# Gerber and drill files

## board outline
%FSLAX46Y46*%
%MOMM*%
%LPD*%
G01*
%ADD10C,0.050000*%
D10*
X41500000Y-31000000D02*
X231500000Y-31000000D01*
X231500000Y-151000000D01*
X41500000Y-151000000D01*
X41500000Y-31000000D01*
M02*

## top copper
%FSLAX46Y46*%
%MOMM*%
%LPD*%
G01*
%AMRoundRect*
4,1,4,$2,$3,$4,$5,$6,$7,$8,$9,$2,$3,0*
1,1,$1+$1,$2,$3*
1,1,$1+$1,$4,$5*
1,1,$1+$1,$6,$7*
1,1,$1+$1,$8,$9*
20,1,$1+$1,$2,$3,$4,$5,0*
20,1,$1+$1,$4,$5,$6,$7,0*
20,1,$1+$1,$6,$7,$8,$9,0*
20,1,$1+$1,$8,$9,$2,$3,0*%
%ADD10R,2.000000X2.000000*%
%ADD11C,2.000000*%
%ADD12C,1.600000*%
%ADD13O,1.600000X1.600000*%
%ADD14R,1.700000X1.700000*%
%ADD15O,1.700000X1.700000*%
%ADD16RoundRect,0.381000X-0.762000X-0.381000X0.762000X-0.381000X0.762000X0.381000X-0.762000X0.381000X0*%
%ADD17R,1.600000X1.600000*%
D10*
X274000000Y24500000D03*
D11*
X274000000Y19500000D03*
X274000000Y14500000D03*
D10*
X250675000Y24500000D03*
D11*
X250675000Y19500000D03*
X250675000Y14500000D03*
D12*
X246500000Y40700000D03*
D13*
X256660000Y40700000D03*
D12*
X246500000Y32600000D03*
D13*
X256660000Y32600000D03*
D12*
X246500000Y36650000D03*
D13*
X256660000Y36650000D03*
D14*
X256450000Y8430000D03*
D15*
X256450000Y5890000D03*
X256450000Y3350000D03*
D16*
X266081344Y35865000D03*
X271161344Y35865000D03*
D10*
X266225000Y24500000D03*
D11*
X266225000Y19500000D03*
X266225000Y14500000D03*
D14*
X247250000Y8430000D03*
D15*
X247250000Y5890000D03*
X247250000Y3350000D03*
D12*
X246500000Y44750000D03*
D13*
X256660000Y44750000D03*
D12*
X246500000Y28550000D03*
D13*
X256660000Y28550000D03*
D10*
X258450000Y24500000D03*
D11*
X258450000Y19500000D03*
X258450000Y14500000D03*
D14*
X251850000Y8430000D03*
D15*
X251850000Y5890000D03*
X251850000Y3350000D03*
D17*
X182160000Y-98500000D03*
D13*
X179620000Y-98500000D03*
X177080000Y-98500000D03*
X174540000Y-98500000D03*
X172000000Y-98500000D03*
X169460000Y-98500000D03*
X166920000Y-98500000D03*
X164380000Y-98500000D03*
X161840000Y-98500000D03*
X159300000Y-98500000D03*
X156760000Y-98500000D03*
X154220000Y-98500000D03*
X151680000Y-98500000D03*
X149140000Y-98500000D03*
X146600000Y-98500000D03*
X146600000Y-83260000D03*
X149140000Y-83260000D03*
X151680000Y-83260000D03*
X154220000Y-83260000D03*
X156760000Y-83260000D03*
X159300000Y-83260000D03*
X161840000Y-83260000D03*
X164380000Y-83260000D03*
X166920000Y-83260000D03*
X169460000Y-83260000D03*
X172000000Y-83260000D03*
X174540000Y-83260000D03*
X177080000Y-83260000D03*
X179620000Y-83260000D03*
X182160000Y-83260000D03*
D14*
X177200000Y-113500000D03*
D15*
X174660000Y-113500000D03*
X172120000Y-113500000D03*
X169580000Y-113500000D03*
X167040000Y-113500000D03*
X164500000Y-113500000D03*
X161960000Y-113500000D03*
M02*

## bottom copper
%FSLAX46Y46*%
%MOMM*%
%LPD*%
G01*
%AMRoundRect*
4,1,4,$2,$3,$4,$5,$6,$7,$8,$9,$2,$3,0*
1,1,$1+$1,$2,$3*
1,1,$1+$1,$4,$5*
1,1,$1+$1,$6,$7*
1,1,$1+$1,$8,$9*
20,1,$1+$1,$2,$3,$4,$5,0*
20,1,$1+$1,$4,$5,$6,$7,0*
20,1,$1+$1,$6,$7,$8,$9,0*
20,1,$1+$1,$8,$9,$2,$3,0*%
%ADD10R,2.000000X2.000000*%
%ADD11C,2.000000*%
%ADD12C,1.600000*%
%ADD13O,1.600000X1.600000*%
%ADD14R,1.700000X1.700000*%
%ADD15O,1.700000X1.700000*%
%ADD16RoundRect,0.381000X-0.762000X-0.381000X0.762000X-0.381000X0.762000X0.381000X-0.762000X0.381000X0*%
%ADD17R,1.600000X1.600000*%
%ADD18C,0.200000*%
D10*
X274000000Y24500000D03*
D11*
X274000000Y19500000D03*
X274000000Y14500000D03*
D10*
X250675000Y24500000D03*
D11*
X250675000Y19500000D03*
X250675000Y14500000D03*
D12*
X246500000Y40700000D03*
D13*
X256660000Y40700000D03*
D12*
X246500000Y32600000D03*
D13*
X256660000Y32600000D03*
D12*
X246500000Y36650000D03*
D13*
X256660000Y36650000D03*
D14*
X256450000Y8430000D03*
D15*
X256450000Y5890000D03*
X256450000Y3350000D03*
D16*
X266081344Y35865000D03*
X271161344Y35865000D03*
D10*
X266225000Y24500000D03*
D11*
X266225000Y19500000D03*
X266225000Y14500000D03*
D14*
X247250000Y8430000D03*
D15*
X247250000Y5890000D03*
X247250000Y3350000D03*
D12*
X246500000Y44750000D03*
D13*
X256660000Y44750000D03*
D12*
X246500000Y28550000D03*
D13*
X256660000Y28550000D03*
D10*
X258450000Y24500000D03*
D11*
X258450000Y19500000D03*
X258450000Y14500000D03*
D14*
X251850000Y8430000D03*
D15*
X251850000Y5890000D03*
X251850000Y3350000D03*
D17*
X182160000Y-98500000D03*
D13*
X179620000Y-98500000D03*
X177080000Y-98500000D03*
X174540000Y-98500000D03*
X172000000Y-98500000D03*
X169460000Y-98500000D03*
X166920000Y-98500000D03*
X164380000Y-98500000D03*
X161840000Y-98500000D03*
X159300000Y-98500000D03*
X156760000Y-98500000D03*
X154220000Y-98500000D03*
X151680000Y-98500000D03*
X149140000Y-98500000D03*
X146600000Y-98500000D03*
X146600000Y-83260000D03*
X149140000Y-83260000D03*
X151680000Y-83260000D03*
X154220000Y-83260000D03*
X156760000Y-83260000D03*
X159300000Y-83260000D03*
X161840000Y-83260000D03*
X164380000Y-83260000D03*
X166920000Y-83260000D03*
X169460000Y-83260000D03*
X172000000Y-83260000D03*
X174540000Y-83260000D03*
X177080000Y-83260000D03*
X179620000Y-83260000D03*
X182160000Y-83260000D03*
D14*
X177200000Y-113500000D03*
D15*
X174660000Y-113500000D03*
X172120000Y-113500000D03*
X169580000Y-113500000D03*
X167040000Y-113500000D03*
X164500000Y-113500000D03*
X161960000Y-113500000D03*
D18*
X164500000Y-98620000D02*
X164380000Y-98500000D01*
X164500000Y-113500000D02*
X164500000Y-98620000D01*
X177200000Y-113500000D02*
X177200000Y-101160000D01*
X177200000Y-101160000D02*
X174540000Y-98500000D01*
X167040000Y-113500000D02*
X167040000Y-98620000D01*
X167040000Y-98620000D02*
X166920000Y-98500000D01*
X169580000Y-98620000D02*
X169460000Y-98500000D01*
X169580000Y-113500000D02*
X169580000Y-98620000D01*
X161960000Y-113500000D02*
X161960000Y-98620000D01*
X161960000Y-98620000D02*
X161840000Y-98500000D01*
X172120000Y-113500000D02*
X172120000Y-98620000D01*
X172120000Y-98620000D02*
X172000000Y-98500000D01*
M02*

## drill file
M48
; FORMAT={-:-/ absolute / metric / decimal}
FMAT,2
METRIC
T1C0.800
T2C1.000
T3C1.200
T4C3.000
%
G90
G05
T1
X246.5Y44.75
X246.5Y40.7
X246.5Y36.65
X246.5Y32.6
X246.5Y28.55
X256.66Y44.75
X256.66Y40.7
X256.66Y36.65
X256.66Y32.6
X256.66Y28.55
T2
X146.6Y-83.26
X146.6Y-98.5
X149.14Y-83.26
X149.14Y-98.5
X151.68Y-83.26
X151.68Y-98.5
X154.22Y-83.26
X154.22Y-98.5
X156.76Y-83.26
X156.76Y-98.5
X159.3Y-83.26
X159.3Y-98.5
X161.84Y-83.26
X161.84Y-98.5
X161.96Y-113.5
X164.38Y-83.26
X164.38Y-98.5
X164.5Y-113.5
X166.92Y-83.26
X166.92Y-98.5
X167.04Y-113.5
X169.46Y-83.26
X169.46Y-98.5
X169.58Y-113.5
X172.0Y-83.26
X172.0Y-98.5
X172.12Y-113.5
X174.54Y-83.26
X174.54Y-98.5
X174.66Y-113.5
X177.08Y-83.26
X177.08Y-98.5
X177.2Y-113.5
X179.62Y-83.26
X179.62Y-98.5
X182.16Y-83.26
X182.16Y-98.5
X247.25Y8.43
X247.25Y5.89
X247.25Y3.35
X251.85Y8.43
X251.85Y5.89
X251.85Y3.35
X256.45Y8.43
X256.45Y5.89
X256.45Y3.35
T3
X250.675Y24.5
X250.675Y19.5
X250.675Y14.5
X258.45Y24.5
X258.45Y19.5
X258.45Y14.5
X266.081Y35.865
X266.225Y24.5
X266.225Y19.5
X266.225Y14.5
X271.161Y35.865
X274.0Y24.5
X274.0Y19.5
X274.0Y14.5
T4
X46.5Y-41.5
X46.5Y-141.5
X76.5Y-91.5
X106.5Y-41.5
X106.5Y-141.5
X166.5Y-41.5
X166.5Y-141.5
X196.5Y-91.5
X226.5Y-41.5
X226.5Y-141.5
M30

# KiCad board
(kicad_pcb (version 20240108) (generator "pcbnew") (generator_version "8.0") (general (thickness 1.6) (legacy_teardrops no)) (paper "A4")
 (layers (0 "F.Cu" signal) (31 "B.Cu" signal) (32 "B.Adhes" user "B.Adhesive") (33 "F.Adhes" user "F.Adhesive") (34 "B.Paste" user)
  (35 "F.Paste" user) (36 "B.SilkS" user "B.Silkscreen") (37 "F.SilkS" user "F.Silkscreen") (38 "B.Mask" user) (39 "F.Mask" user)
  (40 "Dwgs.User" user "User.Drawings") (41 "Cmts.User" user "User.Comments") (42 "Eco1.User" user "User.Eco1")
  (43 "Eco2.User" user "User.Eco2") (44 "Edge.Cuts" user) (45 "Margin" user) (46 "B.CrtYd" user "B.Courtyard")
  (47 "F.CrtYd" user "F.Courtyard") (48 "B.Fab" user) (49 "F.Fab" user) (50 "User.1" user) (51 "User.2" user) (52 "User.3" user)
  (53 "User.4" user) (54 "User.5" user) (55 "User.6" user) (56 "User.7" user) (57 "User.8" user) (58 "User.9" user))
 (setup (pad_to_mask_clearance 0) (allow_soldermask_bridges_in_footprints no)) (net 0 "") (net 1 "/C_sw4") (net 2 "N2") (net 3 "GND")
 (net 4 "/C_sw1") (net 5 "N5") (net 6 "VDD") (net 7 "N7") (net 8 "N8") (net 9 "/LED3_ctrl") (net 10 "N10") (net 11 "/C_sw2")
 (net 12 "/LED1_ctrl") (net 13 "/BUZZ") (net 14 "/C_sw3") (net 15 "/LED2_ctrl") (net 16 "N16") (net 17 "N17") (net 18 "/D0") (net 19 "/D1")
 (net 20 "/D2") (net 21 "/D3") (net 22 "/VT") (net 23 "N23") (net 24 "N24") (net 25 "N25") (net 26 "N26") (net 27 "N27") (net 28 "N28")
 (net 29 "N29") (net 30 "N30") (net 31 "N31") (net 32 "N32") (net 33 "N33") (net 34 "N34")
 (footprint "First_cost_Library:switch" (layer "F.Cu") (at 269 -11.5)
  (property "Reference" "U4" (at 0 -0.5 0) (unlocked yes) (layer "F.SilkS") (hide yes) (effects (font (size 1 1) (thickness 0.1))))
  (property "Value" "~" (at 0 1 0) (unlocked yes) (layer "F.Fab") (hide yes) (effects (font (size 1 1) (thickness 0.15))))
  (pad "1" thru_hole rect (at 5 -13) (size 2 2) (drill 1.2) (layers "*.Cu" "*.Mask") (remove_unused_layers no) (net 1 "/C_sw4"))
  (pad "2" thru_hole circle (at 5 -8) (size 2 2) (drill 1.2) (layers "*.Cu" "*.Mask") (remove_unused_layers no) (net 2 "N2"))
  (pad "3" thru_hole circle (at 5 -3) (size 2 2) (drill 1.2) (layers "*.Cu" "*.Mask") (remove_unused_layers no) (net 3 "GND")))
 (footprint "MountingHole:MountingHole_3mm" (layer "F.Cu") (at 196.5 91.5)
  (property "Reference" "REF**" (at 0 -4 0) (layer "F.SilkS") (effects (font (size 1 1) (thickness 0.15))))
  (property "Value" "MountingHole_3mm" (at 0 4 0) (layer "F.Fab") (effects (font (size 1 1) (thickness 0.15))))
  (pad "" np_thru_hole circle (at 0 0) (size 3 3) (drill 3) (layers "*.Cu" "*.Mask")))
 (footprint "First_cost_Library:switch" (layer "F.Cu") (at 245.675 -11.5)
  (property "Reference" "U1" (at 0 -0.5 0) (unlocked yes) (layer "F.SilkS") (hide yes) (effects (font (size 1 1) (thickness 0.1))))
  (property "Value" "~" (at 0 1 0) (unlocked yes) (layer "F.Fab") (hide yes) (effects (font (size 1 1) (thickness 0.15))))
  (pad "1" thru_hole rect (at 5 -13) (size 2 2) (drill 1.2) (layers "*.Cu" "*.Mask") (remove_unused_layers no) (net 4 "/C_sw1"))
  (pad "2" thru_hole circle (at 5 -8) (size 2 2) (drill 1.2) (layers "*.Cu" "*.Mask") (remove_unused_layers no) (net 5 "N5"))
  (pad "3" thru_hole circle (at 5 -3) (size 2 2) (drill 1.2) (layers "*.Cu" "*.Mask") (remove_unused_layers no) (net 3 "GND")))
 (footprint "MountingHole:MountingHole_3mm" (layer "F.Cu") (at 76.5 91.5)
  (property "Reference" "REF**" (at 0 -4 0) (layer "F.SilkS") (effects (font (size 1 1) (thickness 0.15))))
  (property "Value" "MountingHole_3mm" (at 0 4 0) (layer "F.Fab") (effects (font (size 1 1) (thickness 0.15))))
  (pad "" np_thru_hole circle (at 0 0) (size 3 3) (drill 3) (layers "*.Cu" "*.Mask")))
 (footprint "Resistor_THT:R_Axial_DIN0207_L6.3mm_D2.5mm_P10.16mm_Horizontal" (layer "F.Cu") (at 246.5 -40.7)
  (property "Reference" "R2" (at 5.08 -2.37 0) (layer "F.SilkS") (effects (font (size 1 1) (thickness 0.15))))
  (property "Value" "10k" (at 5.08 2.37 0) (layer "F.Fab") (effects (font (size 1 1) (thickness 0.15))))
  (pad "1" thru_hole circle (at 0 0) (size 1.6 1.6) (drill 0.8) (layers "*.Cu" "*.Mask") (remove_unused_layers no) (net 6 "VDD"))
  (pad "2" thru_hole oval (at 10.16 0) (size 1.6 1.6) (drill 0.8) (layers "*.Cu" "*.Mask") (remove_unused_layers no) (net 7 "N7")))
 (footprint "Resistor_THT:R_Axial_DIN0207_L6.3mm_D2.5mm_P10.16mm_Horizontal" (layer "F.Cu") (at 246.5 -32.6)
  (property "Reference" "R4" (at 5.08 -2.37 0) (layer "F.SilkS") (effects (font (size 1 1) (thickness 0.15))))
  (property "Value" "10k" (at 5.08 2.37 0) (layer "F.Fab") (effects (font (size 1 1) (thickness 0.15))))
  (pad "1" thru_hole circle (at 0 0) (size 1.6 1.6) (drill 0.8) (layers "*.Cu" "*.Mask") (remove_unused_layers no) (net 6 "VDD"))
  (pad "2" thru_hole oval (at 10.16 0) (size 1.6 1.6) (drill 0.8) (layers "*.Cu" "*.Mask") (remove_unused_layers no) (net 2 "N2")))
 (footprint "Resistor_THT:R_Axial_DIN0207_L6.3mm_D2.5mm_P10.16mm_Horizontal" (layer "F.Cu") (at 246.5 -36.65)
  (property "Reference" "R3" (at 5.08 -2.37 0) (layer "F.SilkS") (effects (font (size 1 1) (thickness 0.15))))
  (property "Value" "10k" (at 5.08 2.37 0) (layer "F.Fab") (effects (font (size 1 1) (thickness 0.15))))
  (pad "1" thru_hole circle (at 0 0) (size 1.6 1.6) (drill 0.8) (layers "*.Cu" "*.Mask") (remove_unused_layers no) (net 6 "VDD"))
  (pad "2" thru_hole oval (at 10.16 0) (size 1.6 1.6) (drill 0.8) (layers "*.Cu" "*.Mask") (remove_unused_layers no) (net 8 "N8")))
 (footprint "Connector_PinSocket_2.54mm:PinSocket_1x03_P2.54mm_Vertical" (layer "F.Cu") (at 256.45 -8.43)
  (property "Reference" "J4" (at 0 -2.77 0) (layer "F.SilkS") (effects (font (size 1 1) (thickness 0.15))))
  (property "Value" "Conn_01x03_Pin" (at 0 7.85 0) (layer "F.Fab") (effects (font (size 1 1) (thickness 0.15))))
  (pad "1" thru_hole rect (at 0 0) (size 1.7 1.7) (drill 1) (layers "*.Cu" "*.Mask") (remove_unused_layers no) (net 6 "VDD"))
  (pad "2" thru_hole oval (at 0 2.54) (size 1.7 1.7) (drill 1) (layers "*.Cu" "*.Mask") (remove_unused_layers no) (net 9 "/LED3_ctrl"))
  (pad "3" thru_hole oval (at 0 5.08) (size 1.7 1.7) (drill 1) (layers "*.Cu" "*.Mask") (remove_unused_layers no) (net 3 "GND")))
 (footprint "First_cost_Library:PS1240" (layer "F.Cu") (at 268.621344 -46.025)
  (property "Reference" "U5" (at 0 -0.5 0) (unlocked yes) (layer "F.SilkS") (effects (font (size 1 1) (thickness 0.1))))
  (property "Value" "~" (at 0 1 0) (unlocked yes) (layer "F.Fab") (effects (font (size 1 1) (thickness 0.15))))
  (pad "1" thru_hole roundrect (at -2.54 10.16) (size 2.286 1.524) (drill 1.2) (layers "*.Cu" "*.Mask") (remove_unused_layers no)
   (roundrect_rratio 0.25) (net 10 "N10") (thermal_bridge_angle 45))
  (pad "2" thru_hole roundrect (at 2.54 10.16) (size 2.286 1.524) (drill 1.2) (layers "*.Cu" "*.Mask") (remove_unused_layers no)
   (roundrect_rratio 0.25) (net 3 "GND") (thermal_bridge_angle 45)))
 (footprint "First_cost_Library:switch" (layer "F.Cu") (at 261.225 -11.5)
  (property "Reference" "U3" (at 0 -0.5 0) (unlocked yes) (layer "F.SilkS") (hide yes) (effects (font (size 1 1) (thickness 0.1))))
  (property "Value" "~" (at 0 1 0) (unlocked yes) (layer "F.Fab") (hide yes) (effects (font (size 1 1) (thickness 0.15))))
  (pad "1" thru_hole rect (at 5 -13) (size 2 2) (drill 1.2) (layers "*.Cu" "*.Mask") (remove_unused_layers no) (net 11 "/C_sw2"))
  (pad "2" thru_hole circle (at 5 -8) (size 2 2) (drill 1.2) (layers "*.Cu" "*.Mask") (remove_unused_layers no) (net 8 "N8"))
  (pad "3" thru_hole circle (at 5 -3) (size 2 2) (drill 1.2) (layers "*.Cu" "*.Mask") (remove_unused_layers no) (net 3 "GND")))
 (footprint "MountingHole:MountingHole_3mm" (layer "F.Cu") (at 166.5 141.5)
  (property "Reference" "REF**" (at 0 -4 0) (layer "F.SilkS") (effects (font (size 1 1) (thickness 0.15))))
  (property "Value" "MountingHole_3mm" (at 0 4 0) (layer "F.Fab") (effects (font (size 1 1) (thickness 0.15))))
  (pad "" np_thru_hole circle (at 0 0) (size 3 3) (drill 3) (layers "*.Cu" "*.Mask")))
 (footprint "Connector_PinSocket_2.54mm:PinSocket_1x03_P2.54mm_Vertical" (layer "F.Cu") (at 247.25 -8.43)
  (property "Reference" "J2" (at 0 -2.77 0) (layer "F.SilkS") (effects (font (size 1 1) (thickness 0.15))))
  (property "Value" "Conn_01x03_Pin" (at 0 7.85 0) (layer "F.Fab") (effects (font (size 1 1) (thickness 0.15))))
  (pad "1" thru_hole rect (at 0 0) (size 1.7 1.7) (drill 1) (layers "*.Cu" "*.Mask") (remove_unused_layers no) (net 6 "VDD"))
  (pad "2" thru_hole oval (at 0 2.54) (size 1.7 1.7) (drill 1) (layers "*.Cu" "*.Mask") (remove_unused_layers no) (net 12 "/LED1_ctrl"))
  (pad "3" thru_hole oval (at 0 5.08) (size 1.7 1.7) (drill 1) (layers "*.Cu" "*.Mask") (remove_unused_layers no) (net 3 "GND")))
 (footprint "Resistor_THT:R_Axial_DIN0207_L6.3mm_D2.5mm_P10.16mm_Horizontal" (layer "F.Cu") (at 246.5 -44.75)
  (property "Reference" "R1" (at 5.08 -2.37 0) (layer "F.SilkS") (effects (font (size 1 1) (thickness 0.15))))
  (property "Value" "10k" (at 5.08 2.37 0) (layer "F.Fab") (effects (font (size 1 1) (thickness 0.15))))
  (pad "1" thru_hole circle (at 0 0) (size 1.6 1.6) (drill 0.8) (layers "*.Cu" "*.Mask") (remove_unused_layers no) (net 6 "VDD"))
  (pad "2" thru_hole oval (at 10.16 0) (size 1.6 1.6) (drill 0.8) (layers "*.Cu" "*.Mask") (remove_unused_layers no) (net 5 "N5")))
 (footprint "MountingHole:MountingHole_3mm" (layer "F.Cu") (at 106.5 141.5)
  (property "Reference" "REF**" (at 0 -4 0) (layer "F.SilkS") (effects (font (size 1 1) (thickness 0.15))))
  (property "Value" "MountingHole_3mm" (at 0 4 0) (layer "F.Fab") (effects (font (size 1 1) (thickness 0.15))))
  (pad "" np_thru_hole circle (at 0 0) (size 3 3) (drill 3) (layers "*.Cu" "*.Mask")))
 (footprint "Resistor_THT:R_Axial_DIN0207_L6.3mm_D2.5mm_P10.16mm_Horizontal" (layer "F.Cu") (at 246.5 -28.55)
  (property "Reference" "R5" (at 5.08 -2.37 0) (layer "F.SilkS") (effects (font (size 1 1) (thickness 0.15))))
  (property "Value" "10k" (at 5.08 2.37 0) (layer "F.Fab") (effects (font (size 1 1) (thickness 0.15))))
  (pad "1" thru_hole circle (at 0 0) (size 1.6 1.6) (drill 0.8) (layers "*.Cu" "*.Mask") (remove_unused_layers no) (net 10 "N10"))
  (pad "2" thru_hole oval (at 10.16 0) (size 1.6 1.6) (drill 0.8) (layers "*.Cu" "*.Mask") (remove_unused_layers no) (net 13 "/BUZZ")))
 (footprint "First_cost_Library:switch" (layer "F.Cu") (at 253.45 -11.5)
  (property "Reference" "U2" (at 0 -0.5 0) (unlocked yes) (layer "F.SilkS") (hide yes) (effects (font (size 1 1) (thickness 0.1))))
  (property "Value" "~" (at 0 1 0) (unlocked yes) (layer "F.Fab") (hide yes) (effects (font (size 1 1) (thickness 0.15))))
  (pad "1" thru_hole rect (at 5 -13) (size 2 2) (drill 1.2) (layers "*.Cu" "*.Mask") (remove_unused_layers no) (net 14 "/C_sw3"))
  (pad "2" thru_hole circle (at 5 -8) (size 2 2) (drill 1.2) (layers "*.Cu" "*.Mask") (remove_unused_layers no) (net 7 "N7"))
  (pad "3" thru_hole circle (at 5 -3) (size 2 2) (drill 1.2) (layers "*.Cu" "*.Mask") (remove_unused_layers no) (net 3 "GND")))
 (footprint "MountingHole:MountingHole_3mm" (layer "F.Cu") (at 226.5 41.5)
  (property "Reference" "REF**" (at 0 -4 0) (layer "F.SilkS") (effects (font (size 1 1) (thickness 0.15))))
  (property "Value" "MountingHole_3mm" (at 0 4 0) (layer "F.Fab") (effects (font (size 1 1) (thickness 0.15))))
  (pad "" np_thru_hole circle (at 0 0) (size 3 3) (drill 3) (layers "*.Cu" "*.Mask")))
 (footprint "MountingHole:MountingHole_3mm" (layer "F.Cu") (at 166.5 41.5)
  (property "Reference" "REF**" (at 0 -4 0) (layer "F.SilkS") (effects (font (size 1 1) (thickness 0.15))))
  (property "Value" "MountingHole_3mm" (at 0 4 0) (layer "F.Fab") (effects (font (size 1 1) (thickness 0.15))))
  (pad "" np_thru_hole circle (at 0 0) (size 3 3) (drill 3) (layers "*.Cu" "*.Mask")))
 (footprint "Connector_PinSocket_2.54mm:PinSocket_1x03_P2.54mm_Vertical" (layer "F.Cu") (at 251.85 -8.43)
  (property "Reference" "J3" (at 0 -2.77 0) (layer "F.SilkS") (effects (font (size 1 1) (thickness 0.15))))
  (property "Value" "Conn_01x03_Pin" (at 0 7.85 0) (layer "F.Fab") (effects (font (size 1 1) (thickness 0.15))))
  (pad "1" thru_hole rect (at 0 0) (size 1.7 1.7) (drill 1) (layers "*.Cu" "*.Mask") (remove_unused_layers no) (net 6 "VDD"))
  (pad "2" thru_hole oval (at 0 2.54) (size 1.7 1.7) (drill 1) (layers "*.Cu" "*.Mask") (remove_unused_layers no) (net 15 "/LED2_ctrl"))
  (pad "3" thru_hole oval (at 0 5.08) (size 1.7 1.7) (drill 1) (layers "*.Cu" "*.Mask") (remove_unused_layers no) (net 3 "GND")))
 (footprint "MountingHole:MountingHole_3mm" (layer "F.Cu") (at 46.5 141.5)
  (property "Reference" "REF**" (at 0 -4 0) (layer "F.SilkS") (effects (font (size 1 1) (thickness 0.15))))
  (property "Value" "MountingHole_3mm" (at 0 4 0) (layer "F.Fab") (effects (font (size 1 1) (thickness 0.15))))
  (pad "" np_thru_hole circle (at 0 0) (size 3 3) (drill 3) (layers "*.Cu" "*.Mask")))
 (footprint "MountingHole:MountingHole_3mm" (layer "F.Cu") (at 46.5 41.5)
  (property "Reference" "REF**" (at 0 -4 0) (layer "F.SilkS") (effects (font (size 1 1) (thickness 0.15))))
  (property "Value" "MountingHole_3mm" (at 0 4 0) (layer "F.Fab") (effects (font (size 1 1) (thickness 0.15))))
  (pad "" np_thru_hole circle (at 0 0) (size 3 3) (drill 3) (layers "*.Cu" "*.Mask")))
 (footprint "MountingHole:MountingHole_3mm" (layer "F.Cu") (at 226.5 141.5)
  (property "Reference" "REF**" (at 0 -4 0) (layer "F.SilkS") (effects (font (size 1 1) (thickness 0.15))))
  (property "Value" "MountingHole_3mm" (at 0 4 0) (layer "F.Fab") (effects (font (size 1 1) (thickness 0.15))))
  (pad "" np_thru_hole circle (at 0 0) (size 3 3) (drill 3) (layers "*.Cu" "*.Mask")))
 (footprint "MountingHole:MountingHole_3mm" (layer "F.Cu") (at 106.5 41.5)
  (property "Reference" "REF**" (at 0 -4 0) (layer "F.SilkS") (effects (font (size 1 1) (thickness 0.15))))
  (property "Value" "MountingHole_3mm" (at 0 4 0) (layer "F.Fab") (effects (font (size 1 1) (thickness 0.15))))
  (pad "" np_thru_hole circle (at 0 0) (size 3 3) (drill 3) (layers "*.Cu" "*.Mask")))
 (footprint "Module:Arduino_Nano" (layer "B.Cu") (at 182.16 98.5 90)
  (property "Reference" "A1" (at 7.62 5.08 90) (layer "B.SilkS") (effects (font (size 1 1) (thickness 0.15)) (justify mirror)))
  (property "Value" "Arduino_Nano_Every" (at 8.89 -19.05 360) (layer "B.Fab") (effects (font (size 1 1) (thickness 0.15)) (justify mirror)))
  (pad "1" thru_hole rect (at 0 0 90) (size 1.6 1.6) (drill 1) (layers "*.Cu" "*.Mask") (remove_unused_layers no) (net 13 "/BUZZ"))
  (pad "2" thru_hole oval (at 0 -2.54 90) (size 1.6 1.6) (drill 1) (layers "*.Cu" "*.Mask") (remove_unused_layers no) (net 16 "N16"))
  (pad "3" thru_hole oval (at 0 -5.08 90) (size 1.6 1.6) (drill 1) (layers "*.Cu" "*.Mask") (remove_unused_layers no) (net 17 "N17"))
  (pad "4" thru_hole oval (at 0 -7.62 90) (size 1.6 1.6) (drill 1) (layers "*.Cu" "*.Mask") (remove_unused_layers no) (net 3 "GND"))
  (pad "5" thru_hole oval (at 0 -10.16 90) (size 1.6 1.6) (drill 1) (layers "*.Cu" "*.Mask") (remove_unused_layers no) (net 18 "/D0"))
  (pad "6" thru_hole oval (at 0 -12.7 90) (size 1.6 1.6) (drill 1) (layers "*.Cu" "*.Mask") (remove_unused_layers no) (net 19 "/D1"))
  (pad "7" thru_hole oval (at 0 -15.24 90) (size 1.6 1.6) (drill 1) (layers "*.Cu" "*.Mask") (remove_unused_layers no) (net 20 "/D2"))
  (pad "8" thru_hole oval (at 0 -17.78 90) (size 1.6 1.6) (drill 1) (layers "*.Cu" "*.Mask") (remove_unused_layers no) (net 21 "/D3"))
  (pad "9" thru_hole oval (at 0 -20.32 90) (size 1.6 1.6) (drill 1) (layers "*.Cu" "*.Mask") (remove_unused_layers no) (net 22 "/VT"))
  (pad "10" thru_hole oval (at 0 -22.86 90) (size 1.6 1.6) (drill 1) (layers "*.Cu" "*.Mask") (remove_unused_layers no) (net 4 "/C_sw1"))
  (pad "11" thru_hole oval (at 0 -25.4 90) (size 1.6 1.6) (drill 1) (layers "*.Cu" "*.Mask") (remove_unused_layers no) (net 11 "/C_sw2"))
  (pad "12" thru_hole oval (at 0 -27.94 90) (size 1.6 1.6) (drill 1) (layers "*.Cu" "*.Mask") (remove_unused_layers no) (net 14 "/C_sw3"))
  (pad "13" thru_hole oval (at 0 -30.48 90) (size 1.6 1.6) (drill 1) (layers "*.Cu" "*.Mask") (remove_unused_layers no) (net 1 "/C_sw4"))
  (pad "14" thru_hole oval (at 0 -33.02 90) (size 1.6 1.6) (drill 1) (layers "*.Cu" "*.Mask") (remove_unused_layers no)
   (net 12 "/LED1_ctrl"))
  (pad "15" thru_hole oval (at 0 -35.56 90) (size 1.6 1.6) (drill 1) (layers "*.Cu" "*.Mask") (remove_unused_layers no)
   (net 15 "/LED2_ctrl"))
  (pad "16" thru_hole oval (at 15.24 -35.56 90) (size 1.6 1.6) (drill 1) (layers "*.Cu" "*.Mask") (remove_unused_layers no)
   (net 9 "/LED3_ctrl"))
  (pad "17" thru_hole oval (at 15.24 -33.02 90) (size 1.6 1.6) (drill 1) (layers "*.Cu" "*.Mask") (remove_unused_layers no) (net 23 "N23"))
  (pad "18" thru_hole oval (at 15.24 -30.48 90) (size 1.6 1.6) (drill 1) (layers "*.Cu" "*.Mask") (remove_unused_layers no) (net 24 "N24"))
  (pad "19" thru_hole oval (at 15.24 -27.94 90) (size 1.6 1.6) (drill 1) (layers "*.Cu" "*.Mask") (remove_unused_layers no) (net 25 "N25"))
  (pad "20" thru_hole oval (at 15.24 -25.4 90) (size 1.6 1.6) (drill 1) (layers "*.Cu" "*.Mask") (remove_unused_layers no) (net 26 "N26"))
  (pad "21" thru_hole oval (at 15.24 -22.86 90) (size 1.6 1.6) (drill 1) (layers "*.Cu" "*.Mask") (remove_unused_layers no) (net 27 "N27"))
  (pad "22" thru_hole oval (at 15.24 -20.32 90) (size 1.6 1.6) (drill 1) (layers "*.Cu" "*.Mask") (remove_unused_layers no) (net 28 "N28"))
  (pad "23" thru_hole oval (at 15.24 -17.78 90) (size 1.6 1.6) (drill 1) (layers "*.Cu" "*.Mask") (remove_unused_layers no) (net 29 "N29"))
  (pad "24" thru_hole oval (at 15.24 -15.24 90) (size 1.6 1.6) (drill 1) (layers "*.Cu" "*.Mask") (remove_unused_layers no) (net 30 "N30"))
  (pad "25" thru_hole oval (at 15.24 -12.7 90) (size 1.6 1.6) (drill 1) (layers "*.Cu" "*.Mask") (remove_unused_layers no) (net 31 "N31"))
  (pad "26" thru_hole oval (at 15.24 -10.16 90) (size 1.6 1.6) (drill 1) (layers "*.Cu" "*.Mask") (remove_unused_layers no) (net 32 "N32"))
  (pad "27" thru_hole oval (at 15.24 -7.62 90) (size 1.6 1.6) (drill 1) (layers "*.Cu" "*.Mask") (remove_unused_layers no) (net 6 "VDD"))
  (pad "28" thru_hole oval (at 15.24 -5.08 90) (size 1.6 1.6) (drill 1) (layers "*.Cu" "*.Mask") (remove_unused_layers no) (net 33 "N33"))
  (pad "29" thru_hole oval (at 15.24 -2.54 90) (size 1.6 1.6) (drill 1) (layers "*.Cu" "*.Mask") (remove_unused_layers no) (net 3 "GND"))
  (pad "30" thru_hole oval (at 15.24 0 90) (size 1.6 1.6) (drill 1) (layers "*.Cu" "*.Mask") (remove_unused_layers no) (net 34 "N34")))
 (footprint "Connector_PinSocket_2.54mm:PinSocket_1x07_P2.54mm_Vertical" (layer "B.Cu") (at 177.2 113.5 90)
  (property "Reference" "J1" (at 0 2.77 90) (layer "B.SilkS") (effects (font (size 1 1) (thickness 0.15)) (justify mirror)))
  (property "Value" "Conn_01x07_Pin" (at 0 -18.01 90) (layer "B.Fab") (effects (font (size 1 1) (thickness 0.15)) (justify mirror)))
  (pad "1" thru_hole rect (at 0 0 90) (size 1.7 1.7) (drill 1) (layers "*.Cu" "*.Mask") (remove_unused_layers no) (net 3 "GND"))
  (pad "2" thru_hole oval (at 0 -2.54 90) (size 1.7 1.7) (drill 1) (layers "*.Cu" "*.Mask") (remove_unused_layers no) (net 6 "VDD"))
  (pad "3" thru_hole oval (at 0 -5.08 90) (size 1.7 1.7) (drill 1) (layers "*.Cu" "*.Mask") (remove_unused_layers no) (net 18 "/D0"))
  (pad "4" thru_hole oval (at 0 -7.62 90) (size 1.7 1.7) (drill 1) (layers "*.Cu" "*.Mask") (remove_unused_layers no) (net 19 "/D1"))
  (pad "5" thru_hole oval (at 0 -10.16 90) (size 1.7 1.7) (drill 1) (layers "*.Cu" "*.Mask") (remove_unused_layers no) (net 20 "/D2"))
  (pad "6" thru_hole oval (at 0 -12.7 90) (size 1.7 1.7) (drill 1) (layers "*.Cu" "*.Mask") (remove_unused_layers no) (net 21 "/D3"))
  (pad "7" thru_hole oval (at 0 -15.24 90) (size 1.7 1.7) (drill 1) (layers "*.Cu" "*.Mask") (remove_unused_layers no) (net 22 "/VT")))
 (gr_rect (start 41.5 31) (end 231.5 151) (stroke (width 0.05) (type default)) (fill none) (layer "Edge.Cuts"))
 (segment (start 164.5 98.62) (end 164.38 98.5) (width 0.2) (layer "B.Cu") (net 21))
 (segment (start 164.5 113.5) (end 164.5 98.62) (width 0.2) (layer "B.Cu") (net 21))
 (segment (start 177.2 113.5) (end 177.2 101.16) (width 0.2) (layer "B.Cu") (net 3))
 (segment (start 177.2 101.16) (end 174.54 98.5) (width 0.2) (layer "B.Cu") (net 3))
 (segment (start 167.04 113.5) (end 167.04 98.62) (width 0.2) (layer "B.Cu") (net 20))
 (segment (start 167.04 98.62) (end 166.92 98.5) (width 0.2) (layer "B.Cu") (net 20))
 (segment (start 169.58 98.62) (end 169.46 98.5) (width 0.2) (layer "B.Cu") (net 19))
 (segment (start 169.58 113.5) (end 169.58 98.62) (width 0.2) (layer "B.Cu") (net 19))
 (segment (start 161.96 113.5) (end 161.96 98.62) (width 0.2) (layer "B.Cu") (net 22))
 (segment (start 161.96 98.62) (end 161.84 98.5) (width 0.2) (layer "B.Cu") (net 22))
 (segment (start 172.12 113.5) (end 172.12 98.62) (width 0.2) (layer "B.Cu") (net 18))
 (segment (start 172.12 98.62) (end 172 98.5) (width 0.2) (layer "B.Cu") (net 18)))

